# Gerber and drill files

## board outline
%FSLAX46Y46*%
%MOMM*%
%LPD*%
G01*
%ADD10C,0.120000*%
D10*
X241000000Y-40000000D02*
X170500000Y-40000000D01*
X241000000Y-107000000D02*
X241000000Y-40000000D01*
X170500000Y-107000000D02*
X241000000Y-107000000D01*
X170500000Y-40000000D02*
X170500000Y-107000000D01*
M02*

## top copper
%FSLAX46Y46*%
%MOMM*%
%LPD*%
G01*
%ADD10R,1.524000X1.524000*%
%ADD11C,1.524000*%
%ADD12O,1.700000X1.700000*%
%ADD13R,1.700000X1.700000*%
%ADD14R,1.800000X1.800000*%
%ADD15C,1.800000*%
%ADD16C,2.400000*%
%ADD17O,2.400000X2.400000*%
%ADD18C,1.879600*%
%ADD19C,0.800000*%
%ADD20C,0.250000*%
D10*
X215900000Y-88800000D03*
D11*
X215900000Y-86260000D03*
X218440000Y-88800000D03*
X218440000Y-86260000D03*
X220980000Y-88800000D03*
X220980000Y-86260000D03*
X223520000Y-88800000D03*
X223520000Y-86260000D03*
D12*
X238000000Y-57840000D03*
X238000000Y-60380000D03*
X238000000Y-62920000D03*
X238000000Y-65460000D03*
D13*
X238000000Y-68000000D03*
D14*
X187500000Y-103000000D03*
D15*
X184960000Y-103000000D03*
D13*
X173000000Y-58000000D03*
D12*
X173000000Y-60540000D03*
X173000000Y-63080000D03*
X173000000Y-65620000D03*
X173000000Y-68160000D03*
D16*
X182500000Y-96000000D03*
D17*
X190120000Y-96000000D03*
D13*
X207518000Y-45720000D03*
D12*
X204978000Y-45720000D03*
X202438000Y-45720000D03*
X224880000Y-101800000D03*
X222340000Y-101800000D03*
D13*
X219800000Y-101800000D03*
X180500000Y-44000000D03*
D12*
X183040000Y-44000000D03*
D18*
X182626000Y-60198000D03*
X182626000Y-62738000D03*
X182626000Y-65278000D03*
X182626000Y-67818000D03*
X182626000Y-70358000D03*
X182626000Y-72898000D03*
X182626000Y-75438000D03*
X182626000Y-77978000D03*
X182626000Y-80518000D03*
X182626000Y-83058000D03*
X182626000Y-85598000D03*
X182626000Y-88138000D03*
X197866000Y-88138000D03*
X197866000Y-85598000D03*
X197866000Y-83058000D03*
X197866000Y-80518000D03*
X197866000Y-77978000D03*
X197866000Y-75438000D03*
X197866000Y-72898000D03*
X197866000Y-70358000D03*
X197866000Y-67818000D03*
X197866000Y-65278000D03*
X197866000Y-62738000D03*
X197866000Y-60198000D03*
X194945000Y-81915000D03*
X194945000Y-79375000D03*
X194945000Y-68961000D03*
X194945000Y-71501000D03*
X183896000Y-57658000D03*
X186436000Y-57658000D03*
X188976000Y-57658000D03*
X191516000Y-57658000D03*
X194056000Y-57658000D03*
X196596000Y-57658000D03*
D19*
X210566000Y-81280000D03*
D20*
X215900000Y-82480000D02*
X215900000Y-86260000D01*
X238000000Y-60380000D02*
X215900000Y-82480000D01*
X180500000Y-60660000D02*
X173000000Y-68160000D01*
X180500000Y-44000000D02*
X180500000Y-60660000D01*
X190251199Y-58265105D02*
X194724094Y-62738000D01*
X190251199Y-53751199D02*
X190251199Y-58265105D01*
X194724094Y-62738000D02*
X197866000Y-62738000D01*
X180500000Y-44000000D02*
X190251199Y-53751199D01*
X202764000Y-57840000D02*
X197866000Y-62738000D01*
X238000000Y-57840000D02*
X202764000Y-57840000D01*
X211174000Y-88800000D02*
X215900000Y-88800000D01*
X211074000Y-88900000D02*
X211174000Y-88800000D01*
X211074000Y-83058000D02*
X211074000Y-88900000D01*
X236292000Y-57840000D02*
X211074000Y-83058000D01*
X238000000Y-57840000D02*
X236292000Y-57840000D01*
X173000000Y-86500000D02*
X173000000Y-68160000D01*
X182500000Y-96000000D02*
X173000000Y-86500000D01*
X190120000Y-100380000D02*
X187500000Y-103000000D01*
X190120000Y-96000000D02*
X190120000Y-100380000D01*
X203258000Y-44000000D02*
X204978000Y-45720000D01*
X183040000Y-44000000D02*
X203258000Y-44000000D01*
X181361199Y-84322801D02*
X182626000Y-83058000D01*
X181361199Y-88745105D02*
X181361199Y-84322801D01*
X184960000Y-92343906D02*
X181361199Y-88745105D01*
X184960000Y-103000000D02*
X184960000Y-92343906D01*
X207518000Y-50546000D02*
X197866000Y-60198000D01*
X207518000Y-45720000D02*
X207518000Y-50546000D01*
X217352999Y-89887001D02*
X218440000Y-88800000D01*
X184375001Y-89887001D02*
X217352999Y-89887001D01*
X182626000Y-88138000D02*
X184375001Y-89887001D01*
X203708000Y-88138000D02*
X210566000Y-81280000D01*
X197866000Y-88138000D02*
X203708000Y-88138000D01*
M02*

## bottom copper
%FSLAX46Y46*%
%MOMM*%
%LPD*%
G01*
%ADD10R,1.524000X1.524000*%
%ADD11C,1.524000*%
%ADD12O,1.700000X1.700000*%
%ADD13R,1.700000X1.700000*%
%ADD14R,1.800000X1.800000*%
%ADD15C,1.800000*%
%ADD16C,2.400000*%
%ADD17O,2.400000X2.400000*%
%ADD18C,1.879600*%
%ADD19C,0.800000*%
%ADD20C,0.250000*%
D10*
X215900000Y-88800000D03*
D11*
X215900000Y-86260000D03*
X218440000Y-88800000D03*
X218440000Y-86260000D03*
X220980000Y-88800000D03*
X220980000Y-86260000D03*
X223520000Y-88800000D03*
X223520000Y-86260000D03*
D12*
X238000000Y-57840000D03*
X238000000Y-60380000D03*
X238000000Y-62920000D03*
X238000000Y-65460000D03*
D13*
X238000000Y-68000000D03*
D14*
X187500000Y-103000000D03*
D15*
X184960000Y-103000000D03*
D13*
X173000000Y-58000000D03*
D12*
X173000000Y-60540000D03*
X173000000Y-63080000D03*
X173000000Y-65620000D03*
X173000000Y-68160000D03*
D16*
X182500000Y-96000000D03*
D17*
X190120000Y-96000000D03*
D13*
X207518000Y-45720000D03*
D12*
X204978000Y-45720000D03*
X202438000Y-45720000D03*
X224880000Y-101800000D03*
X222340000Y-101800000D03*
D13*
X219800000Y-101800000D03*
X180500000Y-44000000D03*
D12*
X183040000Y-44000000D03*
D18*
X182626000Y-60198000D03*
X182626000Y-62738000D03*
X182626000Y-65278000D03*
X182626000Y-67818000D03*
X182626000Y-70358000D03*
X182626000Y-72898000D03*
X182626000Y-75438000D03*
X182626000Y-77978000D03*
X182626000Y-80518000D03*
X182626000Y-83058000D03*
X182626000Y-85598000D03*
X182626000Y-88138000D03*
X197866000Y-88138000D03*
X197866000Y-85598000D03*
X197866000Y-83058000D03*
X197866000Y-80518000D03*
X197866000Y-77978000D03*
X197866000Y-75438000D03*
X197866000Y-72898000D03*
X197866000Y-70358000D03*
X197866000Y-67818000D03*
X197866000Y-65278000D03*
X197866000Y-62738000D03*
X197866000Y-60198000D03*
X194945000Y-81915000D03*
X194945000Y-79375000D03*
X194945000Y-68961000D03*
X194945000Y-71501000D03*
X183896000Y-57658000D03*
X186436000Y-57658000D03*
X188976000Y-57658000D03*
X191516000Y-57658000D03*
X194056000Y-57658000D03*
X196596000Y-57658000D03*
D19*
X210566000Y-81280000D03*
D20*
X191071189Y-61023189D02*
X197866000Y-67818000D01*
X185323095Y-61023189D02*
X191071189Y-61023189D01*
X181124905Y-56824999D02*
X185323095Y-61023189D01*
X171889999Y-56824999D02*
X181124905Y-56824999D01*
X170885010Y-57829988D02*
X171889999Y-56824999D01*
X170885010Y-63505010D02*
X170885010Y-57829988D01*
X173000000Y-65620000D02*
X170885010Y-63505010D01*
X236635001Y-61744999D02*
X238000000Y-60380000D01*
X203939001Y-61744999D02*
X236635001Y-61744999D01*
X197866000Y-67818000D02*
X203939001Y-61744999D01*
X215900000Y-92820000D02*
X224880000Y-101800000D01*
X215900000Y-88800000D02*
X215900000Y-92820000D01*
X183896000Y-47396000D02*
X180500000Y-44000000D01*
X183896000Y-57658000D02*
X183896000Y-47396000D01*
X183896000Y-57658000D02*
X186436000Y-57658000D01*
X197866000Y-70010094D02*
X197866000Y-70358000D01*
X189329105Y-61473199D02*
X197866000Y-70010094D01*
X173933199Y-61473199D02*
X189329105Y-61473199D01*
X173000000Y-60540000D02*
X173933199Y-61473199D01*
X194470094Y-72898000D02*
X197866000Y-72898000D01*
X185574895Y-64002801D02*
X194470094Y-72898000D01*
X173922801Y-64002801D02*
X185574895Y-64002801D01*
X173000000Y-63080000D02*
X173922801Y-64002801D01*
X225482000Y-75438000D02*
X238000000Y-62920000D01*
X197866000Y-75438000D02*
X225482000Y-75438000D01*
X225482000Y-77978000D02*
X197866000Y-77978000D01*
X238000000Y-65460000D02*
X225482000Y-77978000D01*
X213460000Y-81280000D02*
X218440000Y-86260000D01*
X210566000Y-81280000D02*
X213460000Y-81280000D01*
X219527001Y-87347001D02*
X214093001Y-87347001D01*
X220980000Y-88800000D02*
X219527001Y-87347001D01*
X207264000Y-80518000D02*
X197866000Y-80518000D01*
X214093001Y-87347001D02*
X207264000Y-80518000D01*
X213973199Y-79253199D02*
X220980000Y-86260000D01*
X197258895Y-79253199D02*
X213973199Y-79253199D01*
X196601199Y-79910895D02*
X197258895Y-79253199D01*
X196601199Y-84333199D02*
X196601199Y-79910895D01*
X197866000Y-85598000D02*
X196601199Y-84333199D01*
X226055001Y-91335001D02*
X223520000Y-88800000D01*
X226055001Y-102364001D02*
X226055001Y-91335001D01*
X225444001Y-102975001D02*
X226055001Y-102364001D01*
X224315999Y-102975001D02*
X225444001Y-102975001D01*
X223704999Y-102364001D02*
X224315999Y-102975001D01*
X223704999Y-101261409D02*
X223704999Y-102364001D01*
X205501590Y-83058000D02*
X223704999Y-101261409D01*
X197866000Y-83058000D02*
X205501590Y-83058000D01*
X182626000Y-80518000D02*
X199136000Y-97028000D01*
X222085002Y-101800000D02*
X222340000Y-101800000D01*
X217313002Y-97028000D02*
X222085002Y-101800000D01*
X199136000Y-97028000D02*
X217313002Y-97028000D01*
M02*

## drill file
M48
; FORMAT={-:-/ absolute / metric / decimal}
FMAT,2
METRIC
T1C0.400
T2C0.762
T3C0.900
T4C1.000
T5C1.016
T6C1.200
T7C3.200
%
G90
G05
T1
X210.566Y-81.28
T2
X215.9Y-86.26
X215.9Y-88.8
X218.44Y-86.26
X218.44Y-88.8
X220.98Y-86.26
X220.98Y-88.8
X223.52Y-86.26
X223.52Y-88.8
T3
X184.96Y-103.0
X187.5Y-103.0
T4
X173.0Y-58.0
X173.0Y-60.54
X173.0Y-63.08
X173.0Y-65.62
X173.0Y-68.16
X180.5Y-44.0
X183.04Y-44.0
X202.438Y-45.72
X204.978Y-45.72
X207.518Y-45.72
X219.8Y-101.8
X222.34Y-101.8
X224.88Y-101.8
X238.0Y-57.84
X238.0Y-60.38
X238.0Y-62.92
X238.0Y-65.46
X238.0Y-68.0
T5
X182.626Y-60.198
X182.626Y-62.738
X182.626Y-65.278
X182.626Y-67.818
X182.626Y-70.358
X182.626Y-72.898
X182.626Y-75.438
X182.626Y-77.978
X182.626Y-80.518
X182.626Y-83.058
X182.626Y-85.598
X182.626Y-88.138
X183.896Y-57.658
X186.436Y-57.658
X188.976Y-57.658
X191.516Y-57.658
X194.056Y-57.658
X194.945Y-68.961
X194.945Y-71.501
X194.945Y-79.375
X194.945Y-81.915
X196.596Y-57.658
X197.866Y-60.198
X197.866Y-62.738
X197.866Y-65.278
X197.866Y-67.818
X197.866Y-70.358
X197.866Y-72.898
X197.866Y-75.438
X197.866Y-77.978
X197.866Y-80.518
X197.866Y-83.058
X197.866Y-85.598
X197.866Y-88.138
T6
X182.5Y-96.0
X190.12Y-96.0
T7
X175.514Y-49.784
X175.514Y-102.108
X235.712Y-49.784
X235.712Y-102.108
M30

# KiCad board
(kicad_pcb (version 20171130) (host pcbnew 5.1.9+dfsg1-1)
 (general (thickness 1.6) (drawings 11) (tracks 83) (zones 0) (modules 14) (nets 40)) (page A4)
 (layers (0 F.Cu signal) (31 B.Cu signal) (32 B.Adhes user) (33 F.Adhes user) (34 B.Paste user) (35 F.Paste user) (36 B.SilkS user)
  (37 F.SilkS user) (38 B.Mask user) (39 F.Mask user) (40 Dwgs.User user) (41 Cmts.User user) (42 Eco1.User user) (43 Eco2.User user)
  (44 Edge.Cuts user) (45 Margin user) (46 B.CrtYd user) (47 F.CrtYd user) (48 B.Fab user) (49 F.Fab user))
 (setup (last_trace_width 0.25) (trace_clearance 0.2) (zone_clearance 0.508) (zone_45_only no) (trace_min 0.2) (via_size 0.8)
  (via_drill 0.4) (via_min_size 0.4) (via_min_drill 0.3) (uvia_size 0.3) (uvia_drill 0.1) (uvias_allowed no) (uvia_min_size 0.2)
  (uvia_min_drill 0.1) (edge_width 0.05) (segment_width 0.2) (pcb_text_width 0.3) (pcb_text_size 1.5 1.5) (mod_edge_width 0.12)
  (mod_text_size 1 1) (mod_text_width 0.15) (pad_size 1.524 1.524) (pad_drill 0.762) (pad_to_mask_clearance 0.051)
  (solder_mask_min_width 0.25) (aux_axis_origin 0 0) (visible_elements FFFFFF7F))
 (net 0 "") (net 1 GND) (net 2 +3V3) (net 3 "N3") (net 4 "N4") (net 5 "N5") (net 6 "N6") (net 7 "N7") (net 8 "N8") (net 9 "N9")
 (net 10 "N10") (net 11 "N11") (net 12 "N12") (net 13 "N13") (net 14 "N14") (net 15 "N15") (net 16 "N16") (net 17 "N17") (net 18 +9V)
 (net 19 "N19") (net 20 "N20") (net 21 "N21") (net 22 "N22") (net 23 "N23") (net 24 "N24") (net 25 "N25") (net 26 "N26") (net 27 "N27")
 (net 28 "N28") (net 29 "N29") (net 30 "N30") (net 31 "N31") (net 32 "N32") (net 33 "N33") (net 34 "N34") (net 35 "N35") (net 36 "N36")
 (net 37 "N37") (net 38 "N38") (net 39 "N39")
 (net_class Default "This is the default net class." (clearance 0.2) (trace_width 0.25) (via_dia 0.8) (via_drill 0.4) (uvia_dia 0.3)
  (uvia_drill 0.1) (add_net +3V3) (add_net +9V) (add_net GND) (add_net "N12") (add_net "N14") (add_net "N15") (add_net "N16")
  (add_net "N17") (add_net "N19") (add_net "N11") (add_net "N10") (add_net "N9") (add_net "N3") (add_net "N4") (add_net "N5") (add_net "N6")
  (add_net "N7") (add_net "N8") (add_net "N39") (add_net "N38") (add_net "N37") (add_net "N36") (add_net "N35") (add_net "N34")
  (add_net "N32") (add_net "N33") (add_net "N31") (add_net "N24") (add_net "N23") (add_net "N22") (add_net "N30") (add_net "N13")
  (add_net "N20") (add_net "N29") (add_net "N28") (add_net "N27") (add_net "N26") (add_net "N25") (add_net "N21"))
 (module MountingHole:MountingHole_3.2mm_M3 (layer F.Cu) (at 235.712 49.784)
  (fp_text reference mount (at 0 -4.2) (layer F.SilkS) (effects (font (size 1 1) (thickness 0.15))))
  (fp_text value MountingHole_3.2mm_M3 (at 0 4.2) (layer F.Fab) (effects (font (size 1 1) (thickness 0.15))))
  (pad 1 np_thru_hole circle (at 0 0) (size 3.2 3.2) (drill 3.2) (layers *.Cu *.Mask)))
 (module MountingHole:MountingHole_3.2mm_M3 (layer F.Cu) (at 175.514 49.784)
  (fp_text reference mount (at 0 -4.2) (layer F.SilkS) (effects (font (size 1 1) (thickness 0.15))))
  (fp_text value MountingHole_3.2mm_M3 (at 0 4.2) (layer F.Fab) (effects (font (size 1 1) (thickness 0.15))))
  (pad 1 np_thru_hole circle (at 0 0) (size 3.2 3.2) (drill 3.2) (layers *.Cu *.Mask)))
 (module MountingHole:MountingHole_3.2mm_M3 (layer F.Cu) (at 175.514 102.108)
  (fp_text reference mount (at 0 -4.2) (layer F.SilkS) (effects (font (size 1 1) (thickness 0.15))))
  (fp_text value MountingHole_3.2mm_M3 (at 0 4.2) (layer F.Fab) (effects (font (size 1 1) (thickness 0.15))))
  (pad 1 np_thru_hole circle (at 0 0) (size 3.2 3.2) (drill 3.2) (layers *.Cu *.Mask)))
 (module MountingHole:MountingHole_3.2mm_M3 (layer F.Cu) (at 235.712 102.108)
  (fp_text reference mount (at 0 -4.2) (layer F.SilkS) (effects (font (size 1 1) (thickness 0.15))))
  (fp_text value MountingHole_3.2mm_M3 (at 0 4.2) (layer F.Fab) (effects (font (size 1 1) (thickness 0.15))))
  (pad 1 np_thru_hole circle (at 0 0) (size 3.2 3.2) (drill 3.2) (layers *.Cu *.Mask)))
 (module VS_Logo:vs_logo (layer B.Cu) (at 204.724 70.612 180)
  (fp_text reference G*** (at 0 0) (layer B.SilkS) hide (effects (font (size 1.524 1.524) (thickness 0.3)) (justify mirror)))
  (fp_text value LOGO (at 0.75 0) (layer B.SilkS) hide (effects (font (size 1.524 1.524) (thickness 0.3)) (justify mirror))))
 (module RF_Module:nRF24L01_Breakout (layer F.Cu) (at 215.9 88.8 90)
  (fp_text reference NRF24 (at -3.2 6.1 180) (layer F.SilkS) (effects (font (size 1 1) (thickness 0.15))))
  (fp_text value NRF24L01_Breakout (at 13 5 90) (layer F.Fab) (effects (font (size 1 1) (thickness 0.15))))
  (pad 1 thru_hole rect (at 0 0 90) (size 1.524 1.524) (drill 0.762) (layers *.Cu *.Mask) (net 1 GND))
  (pad 2 thru_hole circle (at 2.54 0 90) (size 1.524 1.524) (drill 0.762) (layers *.Cu *.Mask) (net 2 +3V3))
  (pad 3 thru_hole circle (at 0 2.54 90) (size 1.524 1.524) (drill 0.762) (layers *.Cu *.Mask) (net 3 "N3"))
  (pad 4 thru_hole circle (at 2.54 2.54 90) (size 1.524 1.524) (drill 0.762) (layers *.Cu *.Mask) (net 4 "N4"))
  (pad 5 thru_hole circle (at 0 5.08 90) (size 1.524 1.524) (drill 0.762) (layers *.Cu *.Mask) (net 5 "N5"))
  (pad 6 thru_hole circle (at 2.54 5.08 90) (size 1.524 1.524) (drill 0.762) (layers *.Cu *.Mask) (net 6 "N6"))
  (pad 7 thru_hole circle (at 0 7.62 90) (size 1.524 1.524) (drill 0.762) (layers *.Cu *.Mask) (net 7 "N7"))
  (pad 8 thru_hole circle (at 2.54 7.62 90) (size 1.524 1.524) (drill 0.762) (layers *.Cu *.Mask) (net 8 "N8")))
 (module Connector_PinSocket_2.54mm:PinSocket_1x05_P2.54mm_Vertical (layer F.Cu) (at 238 68 180)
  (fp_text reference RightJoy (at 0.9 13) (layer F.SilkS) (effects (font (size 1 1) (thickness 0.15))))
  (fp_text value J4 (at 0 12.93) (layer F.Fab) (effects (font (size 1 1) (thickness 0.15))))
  (pad 5 thru_hole oval (at 0 10.16 180) (size 1.7 1.7) (drill 1) (layers *.Cu *.Mask) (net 1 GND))
  (pad 4 thru_hole oval (at 0 7.62 180) (size 1.7 1.7) (drill 1) (layers *.Cu *.Mask) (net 2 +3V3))
  (pad 3 thru_hole oval (at 0 5.08 180) (size 1.7 1.7) (drill 1) (layers *.Cu *.Mask) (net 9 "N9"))
  (pad 2 thru_hole oval (at 0 2.54 180) (size 1.7 1.7) (drill 1) (layers *.Cu *.Mask) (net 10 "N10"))
  (pad 1 thru_hole rect (at 0 0 180) (size 1.7 1.7) (drill 1) (layers *.Cu *.Mask) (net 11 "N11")))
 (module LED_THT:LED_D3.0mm (layer F.Cu) (at 187.5 103 180)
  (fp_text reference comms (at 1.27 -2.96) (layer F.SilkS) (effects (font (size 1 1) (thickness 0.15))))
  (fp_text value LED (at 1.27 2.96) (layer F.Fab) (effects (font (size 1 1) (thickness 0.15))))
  (pad 1 thru_hole rect (at 0 0 180) (size 1.8 1.8) (drill 0.9) (layers *.Cu *.Mask) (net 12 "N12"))
  (pad 2 thru_hole circle (at 2.54 0 180) (size 1.8 1.8) (drill 0.9) (layers *.Cu *.Mask) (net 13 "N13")))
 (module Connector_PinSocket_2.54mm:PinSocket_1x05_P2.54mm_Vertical (layer F.Cu) (at 173 58)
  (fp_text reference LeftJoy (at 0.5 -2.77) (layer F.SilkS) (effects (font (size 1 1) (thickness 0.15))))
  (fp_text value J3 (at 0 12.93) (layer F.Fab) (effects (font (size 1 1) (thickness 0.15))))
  (pad 1 thru_hole rect (at 0 0) (size 1.7 1.7) (drill 1) (layers *.Cu *.Mask) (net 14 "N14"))
  (pad 2 thru_hole oval (at 0 2.54) (size 1.7 1.7) (drill 1) (layers *.Cu *.Mask) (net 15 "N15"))
  (pad 3 thru_hole oval (at 0 5.08) (size 1.7 1.7) (drill 1) (layers *.Cu *.Mask) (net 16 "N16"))
  (pad 4 thru_hole oval (at 0 7.62) (size 1.7 1.7) (drill 1) (layers *.Cu *.Mask) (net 2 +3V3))
  (pad 5 thru_hole oval (at 0 10.16) (size 1.7 1.7) (drill 1) (layers *.Cu *.Mask) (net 1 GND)))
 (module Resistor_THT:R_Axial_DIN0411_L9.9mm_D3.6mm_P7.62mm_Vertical (layer F.Cu) (at 182.5 96)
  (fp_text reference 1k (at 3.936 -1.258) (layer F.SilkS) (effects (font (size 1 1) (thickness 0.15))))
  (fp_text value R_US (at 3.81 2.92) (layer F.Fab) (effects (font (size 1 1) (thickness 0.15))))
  (pad 1 thru_hole circle (at 0 0) (size 2.4 2.4) (drill 1.2) (layers *.Cu *.Mask) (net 1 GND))
  (pad 2 thru_hole oval (at 7.62 0) (size 2.4 2.4) (drill 1.2) (layers *.Cu *.Mask) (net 12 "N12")))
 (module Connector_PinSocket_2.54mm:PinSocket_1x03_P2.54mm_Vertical (layer F.Cu) (at 207.518 45.72 270)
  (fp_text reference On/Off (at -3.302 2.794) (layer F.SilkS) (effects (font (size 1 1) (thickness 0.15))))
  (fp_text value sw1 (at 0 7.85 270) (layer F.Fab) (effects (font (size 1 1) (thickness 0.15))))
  (pad 1 thru_hole rect (at 0 0 270) (size 1.7 1.7) (drill 1) (layers *.Cu *.Mask) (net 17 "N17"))
  (pad 2 thru_hole oval (at 0 2.54 270) (size 1.7 1.7) (drill 1) (layers *.Cu *.Mask) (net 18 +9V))
  (pad 3 thru_hole oval (at 0 5.08 270) (size 1.7 1.7) (drill 1) (layers *.Cu *.Mask) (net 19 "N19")))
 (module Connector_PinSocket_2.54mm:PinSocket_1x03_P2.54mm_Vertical (layer F.Cu) (at 219.8 101.8 90)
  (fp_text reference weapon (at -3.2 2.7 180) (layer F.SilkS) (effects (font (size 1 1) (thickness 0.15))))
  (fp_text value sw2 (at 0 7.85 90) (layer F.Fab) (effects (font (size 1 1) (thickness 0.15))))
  (pad 3 thru_hole oval (at 0 5.08 90) (size 1.7 1.7) (drill 1) (layers *.Cu *.Mask) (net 1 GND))
  (pad 2 thru_hole oval (at 0 2.54 90) (size 1.7 1.7) (drill 1) (layers *.Cu *.Mask) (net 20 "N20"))
  (pad 1 thru_hole rect (at 0 0 90) (size 1.7 1.7) (drill 1) (layers *.Cu *.Mask) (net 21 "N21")))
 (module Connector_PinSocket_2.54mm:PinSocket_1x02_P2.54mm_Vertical (layer F.Cu) (at 180.5 44 90)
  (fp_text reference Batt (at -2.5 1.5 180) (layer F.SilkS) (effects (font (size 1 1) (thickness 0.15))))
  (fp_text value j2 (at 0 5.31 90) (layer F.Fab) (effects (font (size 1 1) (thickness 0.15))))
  (pad 1 thru_hole rect (at 0 0 90) (size 1.7 1.7) (drill 1) (layers *.Cu *.Mask) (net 1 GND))
  (pad 2 thru_hole oval (at 0 2.54 90) (size 1.7 1.7) (drill 1) (layers *.Cu *.Mask) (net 18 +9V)))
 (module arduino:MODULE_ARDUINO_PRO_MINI (layer F.Cu) (at 190.246 72.898)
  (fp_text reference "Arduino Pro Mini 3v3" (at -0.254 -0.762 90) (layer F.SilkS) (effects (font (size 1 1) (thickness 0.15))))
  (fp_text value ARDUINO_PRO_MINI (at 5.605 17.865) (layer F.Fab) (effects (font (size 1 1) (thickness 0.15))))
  (pad JP7_12 thru_hole circle (at -7.62 -12.7) (size 1.8796 1.8796) (drill 1.016) (layers *.Cu *.Mask) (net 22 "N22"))
  (pad JP7_11 thru_hole circle (at -7.62 -10.16) (size 1.8796 1.8796) (drill 1.016) (layers *.Cu *.Mask) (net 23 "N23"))
  (pad JP7_10 thru_hole circle (at -7.62 -7.62) (size 1.8796 1.8796) (drill 1.016) (layers *.Cu *.Mask) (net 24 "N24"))
  (pad JP7_9 thru_hole circle (at -7.62 -5.08) (size 1.8796 1.8796) (drill 1.016) (layers *.Cu *.Mask) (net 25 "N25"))
  (pad JP7_8 thru_hole circle (at -7.62 -2.54) (size 1.8796 1.8796) (drill 1.016) (layers *.Cu *.Mask) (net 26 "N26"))
  (pad JP7_7 thru_hole circle (at -7.62 0) (size 1.8796 1.8796) (drill 1.016) (layers *.Cu *.Mask) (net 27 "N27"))
  (pad JP7_6 thru_hole circle (at -7.62 2.54) (size 1.8796 1.8796) (drill 1.016) (layers *.Cu *.Mask) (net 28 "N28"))
  (pad JP7_5 thru_hole circle (at -7.62 5.08) (size 1.8796 1.8796) (drill 1.016) (layers *.Cu *.Mask) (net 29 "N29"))
  (pad JP7_4 thru_hole circle (at -7.62 7.62) (size 1.8796 1.8796) (drill 1.016) (layers *.Cu *.Mask) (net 20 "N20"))
  (pad JP7_3 thru_hole circle (at -7.62 10.16) (size 1.8796 1.8796) (drill 1.016) (layers *.Cu *.Mask) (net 13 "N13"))
  (pad JP7_2 thru_hole circle (at -7.62 12.7) (size 1.8796 1.8796) (drill 1.016) (layers *.Cu *.Mask) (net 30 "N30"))
  (pad JP7_1 thru_hole circle (at -7.62 15.24) (size 1.8796 1.8796) (drill 1.016) (layers *.Cu *.Mask) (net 3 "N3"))
  (pad JP6_12 thru_hole circle (at 7.62 15.24) (size 1.8796 1.8796) (drill 1.016) (layers *.Cu *.Mask) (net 4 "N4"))
  (pad JP6_11 thru_hole circle (at 7.62 12.7) (size 1.8796 1.8796) (drill 1.016) (layers *.Cu *.Mask) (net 6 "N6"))
  (pad JP6_10 thru_hole circle (at 7.62 10.16) (size 1.8796 1.8796) (drill 1.016) (layers *.Cu *.Mask) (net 7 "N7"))
  (pad JP6_9 thru_hole circle (at 7.62 7.62) (size 1.8796 1.8796) (drill 1.016) (layers *.Cu *.Mask) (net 5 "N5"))
  (pad JP6_8 thru_hole circle (at 7.62 5.08) (size 1.8796 1.8796) (drill 1.016) (layers *.Cu *.Mask) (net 10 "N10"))
  (pad JP6_7 thru_hole circle (at 7.62 2.54) (size 1.8796 1.8796) (drill 1.016) (layers *.Cu *.Mask) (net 9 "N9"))
  (pad JP6_6 thru_hole circle (at 7.62 0) (size 1.8796 1.8796) (drill 1.016) (layers *.Cu *.Mask) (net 16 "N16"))
  (pad JP6_5 thru_hole circle (at 7.62 -2.54) (size 1.8796 1.8796) (drill 1.016) (layers *.Cu *.Mask) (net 15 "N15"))
  (pad JP6_4 thru_hole circle (at 7.62 -5.08) (size 1.8796 1.8796) (drill 1.016) (layers *.Cu *.Mask) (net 2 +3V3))
  (pad JP6_3 thru_hole circle (at 7.62 -7.62) (size 1.8796 1.8796) (drill 1.016) (layers *.Cu *.Mask) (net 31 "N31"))
  (pad JP6_2 thru_hole circle (at 7.62 -10.16) (size 1.8796 1.8796) (drill 1.016) (layers *.Cu *.Mask) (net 1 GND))
  (pad JP6_1 thru_hole circle (at 7.62 -12.7) (size 1.8796 1.8796) (drill 1.016) (layers *.Cu *.Mask) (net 17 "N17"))
  (pad JP3_1 thru_hole circle (at 4.699 9.017) (size 1.8796 1.8796) (drill 1.016) (layers *.Cu *.Mask) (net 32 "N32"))
  (pad JP3_2 thru_hole circle (at 4.699 6.477) (size 1.8796 1.8796) (drill 1.016) (layers *.Cu *.Mask) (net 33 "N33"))
  (pad JP2_2 thru_hole circle (at 4.699 -3.937) (size 1.8796 1.8796) (drill 1.016) (layers *.Cu *.Mask) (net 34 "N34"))
  (pad JP2_1 thru_hole circle (at 4.699 -1.397) (size 1.8796 1.8796) (drill 1.016) (layers *.Cu *.Mask) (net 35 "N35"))
  (pad JP1_6 thru_hole circle (at -6.35 -15.24) (size 1.8796 1.8796) (drill 1.016) (layers *.Cu *.Mask) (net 1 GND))
  (pad JP1_5 thru_hole circle (at -3.81 -15.24) (size 1.8796 1.8796) (drill 1.016) (layers *.Cu *.Mask) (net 1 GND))
  (pad JP1_4 thru_hole circle (at -1.27 -15.24) (size 1.8796 1.8796) (drill 1.016) (layers *.Cu *.Mask) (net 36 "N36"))
  (pad JP1_3 thru_hole circle (at 1.27 -15.24) (size 1.8796 1.8796) (drill 1.016) (layers *.Cu *.Mask) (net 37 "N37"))
  (pad JP1_2 thru_hole circle (at 3.81 -15.24) (size 1.8796 1.8796) (drill 1.016) (layers *.Cu *.Mask) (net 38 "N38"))
  (pad JP1_1 thru_hole circle (at 6.35 -15.24) (size 1.8796 1.8796) (drill 1.016) (layers *.Cu *.Mask) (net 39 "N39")))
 (gr_line (start 241 40) (end 170.5 40) (layer Edge.Cuts) (width 0.12))
 (gr_line (start 241 107) (end 241 40) (layer Edge.Cuts) (width 0.12))
 (gr_line (start 170.5 107) (end 241 107) (layer Edge.Cuts) (width 0.12))
 (gr_line (start 170.5 40) (end 170.5 107) (layer Edge.Cuts) (width 0.12))
 (segment (start 215.9 82.48) (end 215.9 86.26) (width 0.25) (layer F.Cu) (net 2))
 (segment (start 238 60.38) (end 215.9 82.48) (width 0.25) (layer F.Cu) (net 2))
 (segment (start 191.071189 61.023189) (end 197.866 67.818) (width 0.25) (layer B.Cu) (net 2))
 (segment (start 185.323095 61.023189) (end 191.071189 61.023189) (width 0.25) (layer B.Cu) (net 2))
 (segment (start 181.124905 56.824999) (end 185.323095 61.023189) (width 0.25) (layer B.Cu) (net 2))
 (segment (start 171.889999 56.824999) (end 181.124905 56.824999) (width 0.25) (layer B.Cu) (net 2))
 (segment (start 170.88501 57.829988) (end 171.889999 56.824999) (width 0.25) (layer B.Cu) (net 2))
 (segment (start 170.88501 63.50501) (end 170.88501 57.829988) (width 0.25) (layer B.Cu) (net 2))
 (segment (start 173 65.62) (end 170.88501 63.50501) (width 0.25) (layer B.Cu) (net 2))
 (segment (start 236.635001 61.744999) (end 238 60.38) (width 0.25) (layer B.Cu) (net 2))
 (segment (start 203.939001 61.744999) (end 236.635001 61.744999) (width 0.25) (layer B.Cu) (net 2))
 (segment (start 197.866 67.818) (end 203.939001 61.744999) (width 0.25) (layer B.Cu) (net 2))
 (segment (start 180.5 60.66) (end 173 68.16) (width 0.25) (layer F.Cu) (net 1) (status 20))
 (segment (start 180.5 44) (end 180.5 60.66) (width 0.25) (layer F.Cu) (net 1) (status 10))
 (segment (start 190.251199 58.265105) (end 194.724094 62.738) (width 0.25) (layer F.Cu) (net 1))
 (segment (start 190.251199 53.751199) (end 190.251199 58.265105) (width 0.25) (layer F.Cu) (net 1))
 (segment (start 194.724094 62.738) (end 197.866 62.738) (width 0.25) (layer F.Cu) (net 1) (status 20))
 (segment (start 180.5 44) (end 190.251199 53.751199) (width 0.25) (layer F.Cu) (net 1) (status 10))
 (segment (start 202.764 57.84) (end 197.866 62.738) (width 0.25) (layer F.Cu) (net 1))
 (segment (start 238 57.84) (end 202.764 57.84) (width 0.25) (layer F.Cu) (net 1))
 (segment (start 211.174 88.8) (end 215.9 88.8) (width 0.25) (layer F.Cu) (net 1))
 (segment (start 211.074 88.9) (end 211.174 88.8) (width 0.25) (layer F.Cu) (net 1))
 (segment (start 211.074 83.058) (end 211.074 88.9) (width 0.25) (layer F.Cu) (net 1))
 (segment (start 236.292 57.84) (end 211.074 83.058) (width 0.25) (layer F.Cu) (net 1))
 (segment (start 238 57.84) (end 236.292 57.84) (width 0.25) (layer F.Cu) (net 1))
 (segment (start 173 86.5) (end 173 68.16) (width 0.25) (layer F.Cu) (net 1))
 (segment (start 182.5 96) (end 173 86.5) (width 0.25) (layer F.Cu) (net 1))
 (segment (start 215.9 92.82) (end 224.88 101.8) (width 0.25) (layer B.Cu) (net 1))
 (segment (start 215.9 88.8) (end 215.9 92.82) (width 0.25) (layer B.Cu) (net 1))
 (segment (start 183.896 47.396) (end 180.5 44) (width 0.25) (layer B.Cu) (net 1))
 (segment (start 183.896 57.658) (end 183.896 47.396) (width 0.25) (layer B.Cu) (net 1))
 (segment (start 183.896 57.658) (end 186.436 57.658) (width 0.25) (layer B.Cu) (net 1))
 (segment (start 190.12 100.38) (end 187.5 103) (width 0.25) (layer F.Cu) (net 12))
 (segment (start 190.12 96) (end 190.12 100.38) (width 0.25) (layer F.Cu) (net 12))
 (segment (start 203.258 44) (end 204.978 45.72) (width 0.25) (layer F.Cu) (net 18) (status 20))
 (segment (start 183.04 44) (end 203.258 44) (width 0.25) (layer F.Cu) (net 18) (status 10))
 (segment (start 181.361199 84.322801) (end 182.626 83.058) (width 0.25) (layer F.Cu) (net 13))
 (segment (start 181.361199 88.745105) (end 181.361199 84.322801) (width 0.25) (layer F.Cu) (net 13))
 (segment (start 184.96 92.343906) (end 181.361199 88.745105) (width 0.25) (layer F.Cu) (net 13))
 (segment (start 184.96 103) (end 184.96 92.343906) (width 0.25) (layer F.Cu) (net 13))
 (segment (start 197.866 70.010094) (end 197.866 70.358) (width 0.25) (layer B.Cu) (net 15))
 (segment (start 189.329105 61.473199) (end 197.866 70.010094) (width 0.25) (layer B.Cu) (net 15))
 (segment (start 173.933199 61.473199) (end 189.329105 61.473199) (width 0.25) (layer B.Cu) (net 15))
 (segment (start 173 60.54) (end 173.933199 61.473199) (width 0.25) (layer B.Cu) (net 15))
 (segment (start 194.470094 72.898) (end 197.866 72.898) (width 0.25) (layer B.Cu) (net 16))
 (segment (start 185.574895 64.002801) (end 194.470094 72.898) (width 0.25) (layer B.Cu) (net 16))
 (segment (start 173.922801 64.002801) (end 185.574895 64.002801) (width 0.25) (layer B.Cu) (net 16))
 (segment (start 173 63.08) (end 173.922801 64.002801) (width 0.25) (layer B.Cu) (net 16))
 (segment (start 207.518 50.546) (end 197.866 60.198) (width 0.25) (layer F.Cu) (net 17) (status 20))
 (segment (start 207.518 45.72) (end 207.518 50.546) (width 0.25) (layer F.Cu) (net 17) (status 10))
 (segment (start 225.482 75.438) (end 238 62.92) (width 0.25) (layer B.Cu) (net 9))
 (segment (start 197.866 75.438) (end 225.482 75.438) (width 0.25) (layer B.Cu) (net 9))
 (segment (start 225.482 77.978) (end 197.866 77.978) (width 0.25) (layer B.Cu) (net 10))
 (segment (start 238 65.46) (end 225.482 77.978) (width 0.25) (layer B.Cu) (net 10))
 (segment (start 217.352999 89.887001) (end 218.44 88.8) (width 0.25) (layer F.Cu) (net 3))
 (segment (start 184.375001 89.887001) (end 217.352999 89.887001) (width 0.25) (layer F.Cu) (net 3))
 (segment (start 182.626 88.138) (end 184.375001 89.887001) (width 0.25) (layer F.Cu) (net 3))
 (via (at 210.566 81.28) (size 0.8) (drill 0.4) (layers F.Cu B.Cu) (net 4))
 (segment (start 203.708 88.138) (end 210.566 81.28) (width 0.25) (layer F.Cu) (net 4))
 (segment (start 197.866 88.138) (end 203.708 88.138) (width 0.25) (layer F.Cu) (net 4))
 (segment (start 213.46 81.28) (end 218.44 86.26) (width 0.25) (layer B.Cu) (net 4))
 (segment (start 210.566 81.28) (end 213.46 81.28) (width 0.25) (layer B.Cu) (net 4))
 (segment (start 219.527001 87.347001) (end 214.093001 87.347001) (width 0.25) (layer B.Cu) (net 5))
 (segment (start 220.98 88.8) (end 219.527001 87.347001) (width 0.25) (layer B.Cu) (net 5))
 (segment (start 207.264 80.518) (end 197.866 80.518) (width 0.25) (layer B.Cu) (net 5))
 (segment (start 214.093001 87.347001) (end 207.264 80.518) (width 0.25) (layer B.Cu) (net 5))
 (segment (start 213.973199 79.253199) (end 220.98 86.26) (width 0.25) (layer B.Cu) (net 6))
 (segment (start 197.258895 79.253199) (end 213.973199 79.253199) (width 0.25) (layer B.Cu) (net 6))
 (segment (start 196.601199 79.910895) (end 197.258895 79.253199) (width 0.25) (layer B.Cu) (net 6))
 (segment (start 196.601199 84.333199) (end 196.601199 79.910895) (width 0.25) (layer B.Cu) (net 6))
 (segment (start 197.866 85.598) (end 196.601199 84.333199) (width 0.25) (layer B.Cu) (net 6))
 (segment (start 226.055001 91.335001) (end 223.52 88.8) (width 0.25) (layer B.Cu) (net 7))
 (segment (start 226.055001 102.364001) (end 226.055001 91.335001) (width 0.25) (layer B.Cu) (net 7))
 (segment (start 225.444001 102.975001) (end 226.055001 102.364001) (width 0.25) (layer B.Cu) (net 7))
 (segment (start 224.315999 102.975001) (end 225.444001 102.975001) (width 0.25) (layer B.Cu) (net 7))
 (segment (start 223.704999 102.364001) (end 224.315999 102.975001) (width 0.25) (layer B.Cu) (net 7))
 (segment (start 223.704999 101.261409) (end 223.704999 102.364001) (width 0.25) (layer B.Cu) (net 7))
 (segment (start 205.50159 83.058) (end 223.704999 101.261409) (width 0.25) (layer B.Cu) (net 7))
 (segment (start 197.866 83.058) (end 205.50159 83.058) (width 0.25) (layer B.Cu) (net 7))
 (segment (start 182.626 80.518) (end 199.136 97.028) (width 0.25) (layer B.Cu) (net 20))
 (segment (start 222.085002 101.8) (end 222.34 101.8) (width 0.25) (layer B.Cu) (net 20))
 (segment (start 217.313002 97.028) (end 222.085002 101.8) (width 0.25) (layer B.Cu) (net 20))
 (segment (start 199.136 97.028) (end 217.313002 97.028) (width 0.25) (layer B.Cu) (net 20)))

